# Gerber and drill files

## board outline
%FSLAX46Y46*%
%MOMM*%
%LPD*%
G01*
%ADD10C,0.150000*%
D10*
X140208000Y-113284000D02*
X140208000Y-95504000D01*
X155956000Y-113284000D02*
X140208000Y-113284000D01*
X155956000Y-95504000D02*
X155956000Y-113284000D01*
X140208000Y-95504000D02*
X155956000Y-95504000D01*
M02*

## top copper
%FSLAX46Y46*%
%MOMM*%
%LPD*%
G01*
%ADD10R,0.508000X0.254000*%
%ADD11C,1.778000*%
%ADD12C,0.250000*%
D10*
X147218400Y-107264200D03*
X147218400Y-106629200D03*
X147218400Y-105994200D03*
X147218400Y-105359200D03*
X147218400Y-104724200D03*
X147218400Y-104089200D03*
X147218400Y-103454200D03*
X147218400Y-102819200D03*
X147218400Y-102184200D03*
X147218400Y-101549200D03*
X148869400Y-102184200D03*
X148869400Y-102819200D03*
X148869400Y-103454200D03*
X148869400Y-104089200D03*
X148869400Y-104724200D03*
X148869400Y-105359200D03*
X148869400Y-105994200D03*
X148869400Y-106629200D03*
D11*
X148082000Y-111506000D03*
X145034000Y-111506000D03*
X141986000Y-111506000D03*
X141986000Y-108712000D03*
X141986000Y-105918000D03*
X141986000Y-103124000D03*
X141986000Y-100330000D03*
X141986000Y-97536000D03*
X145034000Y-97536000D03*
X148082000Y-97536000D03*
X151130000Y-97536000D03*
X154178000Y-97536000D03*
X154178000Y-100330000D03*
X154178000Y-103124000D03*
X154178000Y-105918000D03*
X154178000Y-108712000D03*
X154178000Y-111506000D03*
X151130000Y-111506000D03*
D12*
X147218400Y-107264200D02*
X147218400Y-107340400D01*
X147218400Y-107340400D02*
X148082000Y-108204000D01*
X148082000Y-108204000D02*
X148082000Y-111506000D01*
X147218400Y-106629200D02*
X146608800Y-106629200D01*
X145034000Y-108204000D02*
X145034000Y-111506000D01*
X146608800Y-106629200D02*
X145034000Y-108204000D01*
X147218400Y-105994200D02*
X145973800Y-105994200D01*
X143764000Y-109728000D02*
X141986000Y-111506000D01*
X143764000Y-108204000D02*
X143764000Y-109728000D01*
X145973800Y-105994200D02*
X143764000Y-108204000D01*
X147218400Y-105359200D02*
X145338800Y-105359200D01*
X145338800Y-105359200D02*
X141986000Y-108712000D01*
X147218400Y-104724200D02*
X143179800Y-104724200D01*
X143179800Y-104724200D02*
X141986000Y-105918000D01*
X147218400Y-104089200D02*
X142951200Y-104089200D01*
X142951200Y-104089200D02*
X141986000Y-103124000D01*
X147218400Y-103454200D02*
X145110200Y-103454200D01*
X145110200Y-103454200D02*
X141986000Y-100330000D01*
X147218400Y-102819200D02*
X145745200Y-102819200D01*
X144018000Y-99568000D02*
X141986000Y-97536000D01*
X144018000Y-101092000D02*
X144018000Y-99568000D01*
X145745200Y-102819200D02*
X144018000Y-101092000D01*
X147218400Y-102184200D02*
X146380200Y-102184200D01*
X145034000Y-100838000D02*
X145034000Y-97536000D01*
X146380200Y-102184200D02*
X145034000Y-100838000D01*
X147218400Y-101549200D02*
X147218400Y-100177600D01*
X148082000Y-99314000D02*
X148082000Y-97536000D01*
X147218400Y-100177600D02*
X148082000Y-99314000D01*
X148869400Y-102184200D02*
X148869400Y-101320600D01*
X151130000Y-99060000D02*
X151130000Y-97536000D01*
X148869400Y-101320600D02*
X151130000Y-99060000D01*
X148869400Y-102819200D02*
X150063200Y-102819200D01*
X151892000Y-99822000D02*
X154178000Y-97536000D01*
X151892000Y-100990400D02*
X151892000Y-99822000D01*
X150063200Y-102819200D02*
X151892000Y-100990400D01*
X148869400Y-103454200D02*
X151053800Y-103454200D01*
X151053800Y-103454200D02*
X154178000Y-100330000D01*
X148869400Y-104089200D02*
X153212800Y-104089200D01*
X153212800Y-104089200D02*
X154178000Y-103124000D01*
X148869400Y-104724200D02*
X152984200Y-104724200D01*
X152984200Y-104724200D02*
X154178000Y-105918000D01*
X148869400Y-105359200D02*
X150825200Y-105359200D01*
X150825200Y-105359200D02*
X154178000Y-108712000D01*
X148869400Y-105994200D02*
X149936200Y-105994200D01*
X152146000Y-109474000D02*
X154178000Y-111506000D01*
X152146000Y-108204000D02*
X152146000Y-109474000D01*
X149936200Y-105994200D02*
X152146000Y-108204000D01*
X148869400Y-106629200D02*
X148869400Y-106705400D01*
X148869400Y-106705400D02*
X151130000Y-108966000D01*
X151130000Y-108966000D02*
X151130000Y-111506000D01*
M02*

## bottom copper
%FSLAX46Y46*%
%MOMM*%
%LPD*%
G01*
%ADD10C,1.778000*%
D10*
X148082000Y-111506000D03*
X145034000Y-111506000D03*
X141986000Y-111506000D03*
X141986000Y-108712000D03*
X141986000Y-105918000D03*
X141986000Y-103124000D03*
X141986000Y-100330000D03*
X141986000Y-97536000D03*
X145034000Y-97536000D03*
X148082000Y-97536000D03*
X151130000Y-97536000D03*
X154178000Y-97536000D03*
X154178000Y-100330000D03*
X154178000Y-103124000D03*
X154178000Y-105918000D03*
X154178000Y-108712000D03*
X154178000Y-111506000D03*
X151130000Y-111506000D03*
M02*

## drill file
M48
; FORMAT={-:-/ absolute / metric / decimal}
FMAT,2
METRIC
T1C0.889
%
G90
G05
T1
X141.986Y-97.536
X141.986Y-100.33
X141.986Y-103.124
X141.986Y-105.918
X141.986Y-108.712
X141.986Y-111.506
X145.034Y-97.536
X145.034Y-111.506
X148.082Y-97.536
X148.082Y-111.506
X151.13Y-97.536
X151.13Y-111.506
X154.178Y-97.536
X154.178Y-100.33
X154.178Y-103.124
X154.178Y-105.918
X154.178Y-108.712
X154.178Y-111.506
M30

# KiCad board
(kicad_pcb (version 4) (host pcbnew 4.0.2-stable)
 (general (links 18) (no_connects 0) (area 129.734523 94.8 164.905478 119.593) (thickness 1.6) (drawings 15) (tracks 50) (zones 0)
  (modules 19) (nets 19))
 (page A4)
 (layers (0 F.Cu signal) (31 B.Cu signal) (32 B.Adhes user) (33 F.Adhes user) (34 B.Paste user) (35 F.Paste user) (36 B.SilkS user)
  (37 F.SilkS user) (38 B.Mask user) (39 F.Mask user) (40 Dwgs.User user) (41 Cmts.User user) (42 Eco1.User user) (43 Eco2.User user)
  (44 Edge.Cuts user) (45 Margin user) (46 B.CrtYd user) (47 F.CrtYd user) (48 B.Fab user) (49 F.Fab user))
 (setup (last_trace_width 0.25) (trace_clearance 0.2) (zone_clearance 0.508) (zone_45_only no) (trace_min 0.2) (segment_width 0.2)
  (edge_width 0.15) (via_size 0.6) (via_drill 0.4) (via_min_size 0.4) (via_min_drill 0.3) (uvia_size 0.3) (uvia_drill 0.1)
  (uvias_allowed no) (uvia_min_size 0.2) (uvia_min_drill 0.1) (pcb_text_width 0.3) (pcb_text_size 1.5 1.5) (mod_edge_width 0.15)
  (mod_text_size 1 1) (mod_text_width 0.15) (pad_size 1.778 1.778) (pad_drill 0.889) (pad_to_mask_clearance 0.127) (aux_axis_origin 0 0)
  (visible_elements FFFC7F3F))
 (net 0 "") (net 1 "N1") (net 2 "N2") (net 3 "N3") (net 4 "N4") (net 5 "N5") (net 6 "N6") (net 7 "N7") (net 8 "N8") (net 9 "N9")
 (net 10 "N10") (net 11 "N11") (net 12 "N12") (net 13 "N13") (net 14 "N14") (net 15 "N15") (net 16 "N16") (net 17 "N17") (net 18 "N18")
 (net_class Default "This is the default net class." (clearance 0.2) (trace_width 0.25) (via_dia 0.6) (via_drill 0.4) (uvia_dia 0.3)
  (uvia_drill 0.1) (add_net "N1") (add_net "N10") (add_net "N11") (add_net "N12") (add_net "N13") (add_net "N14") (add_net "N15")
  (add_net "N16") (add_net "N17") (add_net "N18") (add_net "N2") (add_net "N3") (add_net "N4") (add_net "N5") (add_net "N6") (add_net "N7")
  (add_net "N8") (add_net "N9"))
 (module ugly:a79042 (layer F.Cu) (at 148.082 104.394)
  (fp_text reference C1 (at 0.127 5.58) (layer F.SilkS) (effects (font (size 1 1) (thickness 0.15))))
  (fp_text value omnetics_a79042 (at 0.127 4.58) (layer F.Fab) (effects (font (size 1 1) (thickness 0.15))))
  (pad 1 smd rect (at -0.8636 2.8702) (size 0.508 0.254) (layers F.Cu F.Paste F.Mask) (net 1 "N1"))
  (pad 2 smd rect (at -0.8636 2.2352) (size 0.508 0.254) (layers F.Cu F.Paste F.Mask) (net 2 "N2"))
  (pad 3 smd rect (at -0.8636 1.6002) (size 0.508 0.254) (layers F.Cu F.Paste F.Mask) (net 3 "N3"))
  (pad 4 smd rect (at -0.8636 0.9652) (size 0.508 0.254) (layers F.Cu F.Paste F.Mask) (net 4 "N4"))
  (pad 5 smd rect (at -0.8636 0.3302) (size 0.508 0.254) (layers F.Cu F.Paste F.Mask) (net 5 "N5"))
  (pad 6 smd rect (at -0.8636 -0.3048) (size 0.508 0.254) (layers F.Cu F.Paste F.Mask) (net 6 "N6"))
  (pad 7 smd rect (at -0.8636 -0.9398) (size 0.508 0.254) (layers F.Cu F.Paste F.Mask) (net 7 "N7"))
  (pad 8 smd rect (at -0.8636 -1.5748) (size 0.508 0.254) (layers F.Cu F.Paste F.Mask) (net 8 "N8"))
  (pad 9 smd rect (at -0.8636 -2.2098) (size 0.508 0.254) (layers F.Cu F.Paste F.Mask) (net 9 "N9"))
  (pad 10 smd rect (at -0.8636 -2.8448) (size 0.508 0.254) (layers F.Cu F.Paste F.Mask) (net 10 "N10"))
  (pad 11 smd rect (at 0.7874 -2.2098) (size 0.508 0.254) (layers F.Cu F.Paste F.Mask) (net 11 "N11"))
  (pad 12 smd rect (at 0.7874 -1.5748) (size 0.508 0.254) (layers F.Cu F.Paste F.Mask) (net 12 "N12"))
  (pad 13 smd rect (at 0.7874 -0.9398) (size 0.508 0.254) (layers F.Cu F.Paste F.Mask) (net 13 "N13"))
  (pad 14 smd rect (at 0.7874 -0.3048) (size 0.508 0.254) (layers F.Cu F.Paste F.Mask) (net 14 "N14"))
  (pad 15 smd rect (at 0.7874 0.3302) (size 0.508 0.254) (layers F.Cu F.Paste F.Mask) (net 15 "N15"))
  (pad 16 smd rect (at 0.7874 0.9652) (size 0.508 0.254) (layers F.Cu F.Paste F.Mask) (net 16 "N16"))
  (pad 17 smd rect (at 0.7874 1.6002) (size 0.508 0.254) (layers F.Cu F.Paste F.Mask) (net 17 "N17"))
  (pad 18 smd rect (at 0.7874 2.2352) (size 0.508 0.254) (layers F.Cu F.Paste F.Mask) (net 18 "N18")))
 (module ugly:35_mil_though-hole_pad (layer F.Cu) (at 147.32 114.3)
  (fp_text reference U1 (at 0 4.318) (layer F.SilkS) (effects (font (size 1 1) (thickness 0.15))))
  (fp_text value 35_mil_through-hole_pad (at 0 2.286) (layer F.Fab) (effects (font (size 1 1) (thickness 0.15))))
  (pad 1 thru_hole circle (at 0.762 -2.794) (size 1.778 1.778) (drill 0.889) (layers *.Cu *.Mask F.SilkS) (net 1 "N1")))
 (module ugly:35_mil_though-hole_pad (layer F.Cu) (at 143.51 114.3)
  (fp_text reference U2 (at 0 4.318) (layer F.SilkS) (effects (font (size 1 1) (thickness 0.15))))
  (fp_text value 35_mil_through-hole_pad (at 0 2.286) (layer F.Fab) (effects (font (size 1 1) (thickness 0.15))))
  (pad 1 thru_hole circle (at 1.524 -2.794) (size 1.778 1.778) (drill 0.889) (layers *.Cu *.Mask F.SilkS) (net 2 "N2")))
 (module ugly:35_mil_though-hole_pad (layer F.Cu) (at 139.7 114.3)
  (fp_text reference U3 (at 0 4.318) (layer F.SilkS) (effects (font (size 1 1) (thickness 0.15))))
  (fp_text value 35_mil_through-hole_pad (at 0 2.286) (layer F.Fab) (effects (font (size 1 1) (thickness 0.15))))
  (pad 1 thru_hole circle (at 2.286 -2.794) (size 1.778 1.778) (drill 0.889) (layers *.Cu *.Mask F.SilkS) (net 3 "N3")))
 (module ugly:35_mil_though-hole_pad (layer F.Cu) (at 139.7 110.49)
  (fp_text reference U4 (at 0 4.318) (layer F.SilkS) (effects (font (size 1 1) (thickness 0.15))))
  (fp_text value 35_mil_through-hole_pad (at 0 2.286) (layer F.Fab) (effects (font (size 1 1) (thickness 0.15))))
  (pad 1 thru_hole circle (at 2.286 -1.778) (size 1.778 1.778) (drill 0.889) (layers *.Cu *.Mask F.SilkS) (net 4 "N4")))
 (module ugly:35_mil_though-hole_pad (layer F.Cu) (at 139.7 106.68)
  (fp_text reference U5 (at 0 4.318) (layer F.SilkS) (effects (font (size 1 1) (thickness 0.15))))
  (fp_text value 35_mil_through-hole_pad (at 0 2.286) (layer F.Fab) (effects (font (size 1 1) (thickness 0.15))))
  (pad 1 thru_hole circle (at 2.286 -0.762) (size 1.778 1.778) (drill 0.889) (layers *.Cu *.Mask F.SilkS) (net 5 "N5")))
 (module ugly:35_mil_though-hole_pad (layer F.Cu) (at 139.7 102.87)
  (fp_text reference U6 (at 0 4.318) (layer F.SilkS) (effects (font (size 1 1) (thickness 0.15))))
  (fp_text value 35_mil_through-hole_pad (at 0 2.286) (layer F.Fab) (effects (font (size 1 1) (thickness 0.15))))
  (pad 1 thru_hole circle (at 2.286 0.254) (size 1.778 1.778) (drill 0.889) (layers *.Cu *.Mask F.SilkS) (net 6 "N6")))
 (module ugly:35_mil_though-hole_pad (layer F.Cu) (at 139.7 99.06)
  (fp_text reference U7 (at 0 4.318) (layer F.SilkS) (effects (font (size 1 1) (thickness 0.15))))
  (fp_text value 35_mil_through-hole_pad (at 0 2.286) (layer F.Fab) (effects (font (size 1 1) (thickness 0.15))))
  (pad 1 thru_hole circle (at 2.286 1.27) (size 1.778 1.778) (drill 0.889) (layers *.Cu *.Mask F.SilkS) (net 7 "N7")))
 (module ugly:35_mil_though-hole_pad (layer F.Cu) (at 139.7 95.25)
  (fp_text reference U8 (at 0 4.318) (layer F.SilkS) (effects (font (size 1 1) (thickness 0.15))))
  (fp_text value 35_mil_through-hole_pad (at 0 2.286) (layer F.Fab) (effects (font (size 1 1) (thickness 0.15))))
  (pad 1 thru_hole circle (at 2.286 2.286) (size 1.778 1.778) (drill 0.889) (layers *.Cu *.Mask F.SilkS) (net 8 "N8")))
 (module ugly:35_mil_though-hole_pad (layer F.Cu) (at 143.51 95.25)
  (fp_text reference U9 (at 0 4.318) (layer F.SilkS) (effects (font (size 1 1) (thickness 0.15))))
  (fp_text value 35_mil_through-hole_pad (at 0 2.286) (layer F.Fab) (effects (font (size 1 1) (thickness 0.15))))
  (pad 1 thru_hole circle (at 1.524 2.286) (size 1.778 1.778) (drill 0.889) (layers *.Cu *.Mask F.SilkS) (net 9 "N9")))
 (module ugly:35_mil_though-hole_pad (layer F.Cu) (at 147.32 95.25)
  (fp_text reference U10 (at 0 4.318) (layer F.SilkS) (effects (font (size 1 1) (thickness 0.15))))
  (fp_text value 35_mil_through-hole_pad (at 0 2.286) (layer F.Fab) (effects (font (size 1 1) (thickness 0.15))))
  (pad 1 thru_hole circle (at 0.762 2.286) (size 1.778 1.778) (drill 0.889) (layers *.Cu *.Mask F.SilkS) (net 10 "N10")))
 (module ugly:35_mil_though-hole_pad (layer F.Cu) (at 151.13 95.25)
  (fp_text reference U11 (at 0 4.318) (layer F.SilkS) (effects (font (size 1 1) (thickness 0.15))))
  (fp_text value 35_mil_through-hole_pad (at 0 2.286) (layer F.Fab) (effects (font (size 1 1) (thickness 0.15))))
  (pad 1 thru_hole circle (at 0 2.286) (size 1.778 1.778) (drill 0.889) (layers *.Cu *.Mask F.SilkS) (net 11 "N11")))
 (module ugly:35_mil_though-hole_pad (layer F.Cu) (at 154.94 95.25)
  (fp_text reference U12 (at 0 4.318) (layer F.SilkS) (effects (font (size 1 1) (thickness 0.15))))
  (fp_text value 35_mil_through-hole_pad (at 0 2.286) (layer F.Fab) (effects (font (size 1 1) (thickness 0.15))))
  (pad 1 thru_hole circle (at -0.762 2.286) (size 1.778 1.778) (drill 0.889) (layers *.Cu *.Mask F.SilkS) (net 12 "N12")))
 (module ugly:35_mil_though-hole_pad (layer F.Cu) (at 154.94 99.06)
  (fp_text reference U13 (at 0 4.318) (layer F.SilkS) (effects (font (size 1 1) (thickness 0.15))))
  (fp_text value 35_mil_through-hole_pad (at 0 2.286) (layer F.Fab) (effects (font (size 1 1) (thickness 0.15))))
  (pad 1 thru_hole circle (at -0.762 1.27) (size 1.778 1.778) (drill 0.889) (layers *.Cu *.Mask F.SilkS) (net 13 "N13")))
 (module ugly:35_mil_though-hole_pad (layer F.Cu) (at 154.94 102.87)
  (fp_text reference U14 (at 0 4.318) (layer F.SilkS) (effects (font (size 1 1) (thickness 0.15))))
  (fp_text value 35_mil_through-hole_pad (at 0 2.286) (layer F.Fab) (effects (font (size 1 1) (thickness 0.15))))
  (pad 1 thru_hole circle (at -0.762 0.254) (size 1.778 1.778) (drill 0.889) (layers *.Cu *.Mask F.SilkS) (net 14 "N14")))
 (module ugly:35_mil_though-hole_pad (layer F.Cu) (at 154.94 106.68)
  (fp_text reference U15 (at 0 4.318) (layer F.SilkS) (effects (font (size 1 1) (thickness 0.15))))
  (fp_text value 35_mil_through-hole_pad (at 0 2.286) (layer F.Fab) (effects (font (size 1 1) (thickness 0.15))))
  (pad 1 thru_hole circle (at -0.762 -0.762) (size 1.778 1.778) (drill 0.889) (layers *.Cu *.Mask F.SilkS) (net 15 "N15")))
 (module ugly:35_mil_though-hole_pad (layer F.Cu) (at 154.94 110.49)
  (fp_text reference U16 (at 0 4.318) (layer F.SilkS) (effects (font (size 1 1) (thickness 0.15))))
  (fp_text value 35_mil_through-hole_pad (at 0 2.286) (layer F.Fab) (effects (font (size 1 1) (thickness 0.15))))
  (pad 1 thru_hole circle (at -0.762 -1.778) (size 1.778 1.778) (drill 0.889) (layers *.Cu *.Mask F.SilkS) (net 16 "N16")))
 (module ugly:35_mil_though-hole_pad (layer F.Cu) (at 154.94 114.3)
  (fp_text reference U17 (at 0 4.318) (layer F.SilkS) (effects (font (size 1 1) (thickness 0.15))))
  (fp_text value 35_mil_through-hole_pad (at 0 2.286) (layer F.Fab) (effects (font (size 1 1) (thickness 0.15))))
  (pad 1 thru_hole circle (at -0.762 -2.794) (size 1.778 1.778) (drill 0.889) (layers *.Cu *.Mask F.SilkS) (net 17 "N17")))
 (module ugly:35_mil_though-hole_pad (layer F.Cu) (at 151.13 114.046)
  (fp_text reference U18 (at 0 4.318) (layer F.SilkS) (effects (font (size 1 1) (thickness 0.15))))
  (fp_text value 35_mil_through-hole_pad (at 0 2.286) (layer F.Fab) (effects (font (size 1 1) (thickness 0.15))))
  (pad 1 thru_hole circle (at 0 -2.54) (size 1.778 1.778) (drill 0.889) (layers *.Cu *.Mask F.SilkS) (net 18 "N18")))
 (gr_line (start 140.208 113.284) (end 140.208 95.504) (angle 90) (layer Edge.Cuts) (width 0.15))
 (gr_line (start 155.956 113.284) (end 140.208 113.284) (angle 90) (layer Edge.Cuts) (width 0.15))
 (gr_line (start 155.956 95.504) (end 155.956 113.284) (angle 90) (layer Edge.Cuts) (width 0.15))
 (gr_line (start 140.208 95.504) (end 155.956 95.504) (angle 90) (layer Edge.Cuts) (width 0.15))
 (segment (start 147.2184 107.2642) (end 147.2184 107.3404) (width 0.25) (layer F.Cu) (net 1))
 (segment (start 147.2184 107.3404) (end 148.082 108.204) (width 0.25) (layer F.Cu) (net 1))
 (segment (start 148.082 108.204) (end 148.082 111.506) (width 0.25) (layer F.Cu) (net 1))
 (segment (start 147.2184 106.6292) (end 146.6088 106.6292) (width 0.25) (layer F.Cu) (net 2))
 (segment (start 145.034 108.204) (end 145.034 111.506) (width 0.25) (layer F.Cu) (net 2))
 (segment (start 146.6088 106.6292) (end 145.034 108.204) (width 0.25) (layer F.Cu) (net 2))
 (segment (start 147.2184 105.9942) (end 145.9738 105.9942) (width 0.25) (layer F.Cu) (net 3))
 (segment (start 143.764 109.728) (end 141.986 111.506) (width 0.25) (layer F.Cu) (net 3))
 (segment (start 143.764 108.204) (end 143.764 109.728) (width 0.25) (layer F.Cu) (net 3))
 (segment (start 145.9738 105.9942) (end 143.764 108.204) (width 0.25) (layer F.Cu) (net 3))
 (segment (start 147.2184 105.3592) (end 145.3388 105.3592) (width 0.25) (layer F.Cu) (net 4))
 (segment (start 145.3388 105.3592) (end 141.986 108.712) (width 0.25) (layer F.Cu) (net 4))
 (segment (start 147.2184 104.7242) (end 143.1798 104.7242) (width 0.25) (layer F.Cu) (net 5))
 (segment (start 143.1798 104.7242) (end 141.986 105.918) (width 0.25) (layer F.Cu) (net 5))
 (segment (start 147.2184 104.0892) (end 142.9512 104.0892) (width 0.25) (layer F.Cu) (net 6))
 (segment (start 142.9512 104.0892) (end 141.986 103.124) (width 0.25) (layer F.Cu) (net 6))
 (segment (start 147.2184 103.4542) (end 145.1102 103.4542) (width 0.25) (layer F.Cu) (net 7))
 (segment (start 145.1102 103.4542) (end 141.986 100.33) (width 0.25) (layer F.Cu) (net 7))
 (segment (start 147.2184 102.8192) (end 145.7452 102.8192) (width 0.25) (layer F.Cu) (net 8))
 (segment (start 144.018 99.568) (end 141.986 97.536) (width 0.25) (layer F.Cu) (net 8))
 (segment (start 144.018 101.092) (end 144.018 99.568) (width 0.25) (layer F.Cu) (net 8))
 (segment (start 145.7452 102.8192) (end 144.018 101.092) (width 0.25) (layer F.Cu) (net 8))
 (segment (start 147.2184 102.1842) (end 146.3802 102.1842) (width 0.25) (layer F.Cu) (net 9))
 (segment (start 145.034 100.838) (end 145.034 97.536) (width 0.25) (layer F.Cu) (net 9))
 (segment (start 146.3802 102.1842) (end 145.034 100.838) (width 0.25) (layer F.Cu) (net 9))
 (segment (start 147.2184 101.5492) (end 147.2184 100.1776) (width 0.25) (layer F.Cu) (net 10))
 (segment (start 148.082 99.314) (end 148.082 97.536) (width 0.25) (layer F.Cu) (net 10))
 (segment (start 147.2184 100.1776) (end 148.082 99.314) (width 0.25) (layer F.Cu) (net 10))
 (segment (start 148.8694 102.1842) (end 148.8694 101.3206) (width 0.25) (layer F.Cu) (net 11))
 (segment (start 151.13 99.06) (end 151.13 97.536) (width 0.25) (layer F.Cu) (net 11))
 (segment (start 148.8694 101.3206) (end 151.13 99.06) (width 0.25) (layer F.Cu) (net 11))
 (segment (start 148.8694 102.8192) (end 150.0632 102.8192) (width 0.25) (layer F.Cu) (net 12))
 (segment (start 151.892 99.822) (end 154.178 97.536) (width 0.25) (layer F.Cu) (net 12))
 (segment (start 151.892 100.9904) (end 151.892 99.822) (width 0.25) (layer F.Cu) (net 12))
 (segment (start 150.0632 102.8192) (end 151.892 100.9904) (width 0.25) (layer F.Cu) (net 12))
 (segment (start 148.8694 103.4542) (end 151.0538 103.4542) (width 0.25) (layer F.Cu) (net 13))
 (segment (start 151.0538 103.4542) (end 154.178 100.33) (width 0.25) (layer F.Cu) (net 13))
 (segment (start 148.8694 104.0892) (end 153.2128 104.0892) (width 0.25) (layer F.Cu) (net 14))
 (segment (start 153.2128 104.0892) (end 154.178 103.124) (width 0.25) (layer F.Cu) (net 14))
 (segment (start 148.8694 104.7242) (end 152.9842 104.7242) (width 0.25) (layer F.Cu) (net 15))
 (segment (start 152.9842 104.7242) (end 154.178 105.918) (width 0.25) (layer F.Cu) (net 15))
 (segment (start 148.8694 105.3592) (end 150.8252 105.3592) (width 0.25) (layer F.Cu) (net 16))
 (segment (start 150.8252 105.3592) (end 154.178 108.712) (width 0.25) (layer F.Cu) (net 16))
 (segment (start 148.8694 105.9942) (end 149.9362 105.9942) (width 0.25) (layer F.Cu) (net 17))
 (segment (start 152.146 109.474) (end 154.178 111.506) (width 0.25) (layer F.Cu) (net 17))
 (segment (start 152.146 108.204) (end 152.146 109.474) (width 0.25) (layer F.Cu) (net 17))
 (segment (start 149.9362 105.9942) (end 152.146 108.204) (width 0.25) (layer F.Cu) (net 17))
 (segment (start 148.8694 106.6292) (end 148.8694 106.7054) (width 0.25) (layer F.Cu) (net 18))
 (segment (start 148.8694 106.7054) (end 151.13 108.966) (width 0.25) (layer F.Cu) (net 18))
 (segment (start 151.13 108.966) (end 151.13 111.506) (width 0.25) (layer F.Cu) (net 18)))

